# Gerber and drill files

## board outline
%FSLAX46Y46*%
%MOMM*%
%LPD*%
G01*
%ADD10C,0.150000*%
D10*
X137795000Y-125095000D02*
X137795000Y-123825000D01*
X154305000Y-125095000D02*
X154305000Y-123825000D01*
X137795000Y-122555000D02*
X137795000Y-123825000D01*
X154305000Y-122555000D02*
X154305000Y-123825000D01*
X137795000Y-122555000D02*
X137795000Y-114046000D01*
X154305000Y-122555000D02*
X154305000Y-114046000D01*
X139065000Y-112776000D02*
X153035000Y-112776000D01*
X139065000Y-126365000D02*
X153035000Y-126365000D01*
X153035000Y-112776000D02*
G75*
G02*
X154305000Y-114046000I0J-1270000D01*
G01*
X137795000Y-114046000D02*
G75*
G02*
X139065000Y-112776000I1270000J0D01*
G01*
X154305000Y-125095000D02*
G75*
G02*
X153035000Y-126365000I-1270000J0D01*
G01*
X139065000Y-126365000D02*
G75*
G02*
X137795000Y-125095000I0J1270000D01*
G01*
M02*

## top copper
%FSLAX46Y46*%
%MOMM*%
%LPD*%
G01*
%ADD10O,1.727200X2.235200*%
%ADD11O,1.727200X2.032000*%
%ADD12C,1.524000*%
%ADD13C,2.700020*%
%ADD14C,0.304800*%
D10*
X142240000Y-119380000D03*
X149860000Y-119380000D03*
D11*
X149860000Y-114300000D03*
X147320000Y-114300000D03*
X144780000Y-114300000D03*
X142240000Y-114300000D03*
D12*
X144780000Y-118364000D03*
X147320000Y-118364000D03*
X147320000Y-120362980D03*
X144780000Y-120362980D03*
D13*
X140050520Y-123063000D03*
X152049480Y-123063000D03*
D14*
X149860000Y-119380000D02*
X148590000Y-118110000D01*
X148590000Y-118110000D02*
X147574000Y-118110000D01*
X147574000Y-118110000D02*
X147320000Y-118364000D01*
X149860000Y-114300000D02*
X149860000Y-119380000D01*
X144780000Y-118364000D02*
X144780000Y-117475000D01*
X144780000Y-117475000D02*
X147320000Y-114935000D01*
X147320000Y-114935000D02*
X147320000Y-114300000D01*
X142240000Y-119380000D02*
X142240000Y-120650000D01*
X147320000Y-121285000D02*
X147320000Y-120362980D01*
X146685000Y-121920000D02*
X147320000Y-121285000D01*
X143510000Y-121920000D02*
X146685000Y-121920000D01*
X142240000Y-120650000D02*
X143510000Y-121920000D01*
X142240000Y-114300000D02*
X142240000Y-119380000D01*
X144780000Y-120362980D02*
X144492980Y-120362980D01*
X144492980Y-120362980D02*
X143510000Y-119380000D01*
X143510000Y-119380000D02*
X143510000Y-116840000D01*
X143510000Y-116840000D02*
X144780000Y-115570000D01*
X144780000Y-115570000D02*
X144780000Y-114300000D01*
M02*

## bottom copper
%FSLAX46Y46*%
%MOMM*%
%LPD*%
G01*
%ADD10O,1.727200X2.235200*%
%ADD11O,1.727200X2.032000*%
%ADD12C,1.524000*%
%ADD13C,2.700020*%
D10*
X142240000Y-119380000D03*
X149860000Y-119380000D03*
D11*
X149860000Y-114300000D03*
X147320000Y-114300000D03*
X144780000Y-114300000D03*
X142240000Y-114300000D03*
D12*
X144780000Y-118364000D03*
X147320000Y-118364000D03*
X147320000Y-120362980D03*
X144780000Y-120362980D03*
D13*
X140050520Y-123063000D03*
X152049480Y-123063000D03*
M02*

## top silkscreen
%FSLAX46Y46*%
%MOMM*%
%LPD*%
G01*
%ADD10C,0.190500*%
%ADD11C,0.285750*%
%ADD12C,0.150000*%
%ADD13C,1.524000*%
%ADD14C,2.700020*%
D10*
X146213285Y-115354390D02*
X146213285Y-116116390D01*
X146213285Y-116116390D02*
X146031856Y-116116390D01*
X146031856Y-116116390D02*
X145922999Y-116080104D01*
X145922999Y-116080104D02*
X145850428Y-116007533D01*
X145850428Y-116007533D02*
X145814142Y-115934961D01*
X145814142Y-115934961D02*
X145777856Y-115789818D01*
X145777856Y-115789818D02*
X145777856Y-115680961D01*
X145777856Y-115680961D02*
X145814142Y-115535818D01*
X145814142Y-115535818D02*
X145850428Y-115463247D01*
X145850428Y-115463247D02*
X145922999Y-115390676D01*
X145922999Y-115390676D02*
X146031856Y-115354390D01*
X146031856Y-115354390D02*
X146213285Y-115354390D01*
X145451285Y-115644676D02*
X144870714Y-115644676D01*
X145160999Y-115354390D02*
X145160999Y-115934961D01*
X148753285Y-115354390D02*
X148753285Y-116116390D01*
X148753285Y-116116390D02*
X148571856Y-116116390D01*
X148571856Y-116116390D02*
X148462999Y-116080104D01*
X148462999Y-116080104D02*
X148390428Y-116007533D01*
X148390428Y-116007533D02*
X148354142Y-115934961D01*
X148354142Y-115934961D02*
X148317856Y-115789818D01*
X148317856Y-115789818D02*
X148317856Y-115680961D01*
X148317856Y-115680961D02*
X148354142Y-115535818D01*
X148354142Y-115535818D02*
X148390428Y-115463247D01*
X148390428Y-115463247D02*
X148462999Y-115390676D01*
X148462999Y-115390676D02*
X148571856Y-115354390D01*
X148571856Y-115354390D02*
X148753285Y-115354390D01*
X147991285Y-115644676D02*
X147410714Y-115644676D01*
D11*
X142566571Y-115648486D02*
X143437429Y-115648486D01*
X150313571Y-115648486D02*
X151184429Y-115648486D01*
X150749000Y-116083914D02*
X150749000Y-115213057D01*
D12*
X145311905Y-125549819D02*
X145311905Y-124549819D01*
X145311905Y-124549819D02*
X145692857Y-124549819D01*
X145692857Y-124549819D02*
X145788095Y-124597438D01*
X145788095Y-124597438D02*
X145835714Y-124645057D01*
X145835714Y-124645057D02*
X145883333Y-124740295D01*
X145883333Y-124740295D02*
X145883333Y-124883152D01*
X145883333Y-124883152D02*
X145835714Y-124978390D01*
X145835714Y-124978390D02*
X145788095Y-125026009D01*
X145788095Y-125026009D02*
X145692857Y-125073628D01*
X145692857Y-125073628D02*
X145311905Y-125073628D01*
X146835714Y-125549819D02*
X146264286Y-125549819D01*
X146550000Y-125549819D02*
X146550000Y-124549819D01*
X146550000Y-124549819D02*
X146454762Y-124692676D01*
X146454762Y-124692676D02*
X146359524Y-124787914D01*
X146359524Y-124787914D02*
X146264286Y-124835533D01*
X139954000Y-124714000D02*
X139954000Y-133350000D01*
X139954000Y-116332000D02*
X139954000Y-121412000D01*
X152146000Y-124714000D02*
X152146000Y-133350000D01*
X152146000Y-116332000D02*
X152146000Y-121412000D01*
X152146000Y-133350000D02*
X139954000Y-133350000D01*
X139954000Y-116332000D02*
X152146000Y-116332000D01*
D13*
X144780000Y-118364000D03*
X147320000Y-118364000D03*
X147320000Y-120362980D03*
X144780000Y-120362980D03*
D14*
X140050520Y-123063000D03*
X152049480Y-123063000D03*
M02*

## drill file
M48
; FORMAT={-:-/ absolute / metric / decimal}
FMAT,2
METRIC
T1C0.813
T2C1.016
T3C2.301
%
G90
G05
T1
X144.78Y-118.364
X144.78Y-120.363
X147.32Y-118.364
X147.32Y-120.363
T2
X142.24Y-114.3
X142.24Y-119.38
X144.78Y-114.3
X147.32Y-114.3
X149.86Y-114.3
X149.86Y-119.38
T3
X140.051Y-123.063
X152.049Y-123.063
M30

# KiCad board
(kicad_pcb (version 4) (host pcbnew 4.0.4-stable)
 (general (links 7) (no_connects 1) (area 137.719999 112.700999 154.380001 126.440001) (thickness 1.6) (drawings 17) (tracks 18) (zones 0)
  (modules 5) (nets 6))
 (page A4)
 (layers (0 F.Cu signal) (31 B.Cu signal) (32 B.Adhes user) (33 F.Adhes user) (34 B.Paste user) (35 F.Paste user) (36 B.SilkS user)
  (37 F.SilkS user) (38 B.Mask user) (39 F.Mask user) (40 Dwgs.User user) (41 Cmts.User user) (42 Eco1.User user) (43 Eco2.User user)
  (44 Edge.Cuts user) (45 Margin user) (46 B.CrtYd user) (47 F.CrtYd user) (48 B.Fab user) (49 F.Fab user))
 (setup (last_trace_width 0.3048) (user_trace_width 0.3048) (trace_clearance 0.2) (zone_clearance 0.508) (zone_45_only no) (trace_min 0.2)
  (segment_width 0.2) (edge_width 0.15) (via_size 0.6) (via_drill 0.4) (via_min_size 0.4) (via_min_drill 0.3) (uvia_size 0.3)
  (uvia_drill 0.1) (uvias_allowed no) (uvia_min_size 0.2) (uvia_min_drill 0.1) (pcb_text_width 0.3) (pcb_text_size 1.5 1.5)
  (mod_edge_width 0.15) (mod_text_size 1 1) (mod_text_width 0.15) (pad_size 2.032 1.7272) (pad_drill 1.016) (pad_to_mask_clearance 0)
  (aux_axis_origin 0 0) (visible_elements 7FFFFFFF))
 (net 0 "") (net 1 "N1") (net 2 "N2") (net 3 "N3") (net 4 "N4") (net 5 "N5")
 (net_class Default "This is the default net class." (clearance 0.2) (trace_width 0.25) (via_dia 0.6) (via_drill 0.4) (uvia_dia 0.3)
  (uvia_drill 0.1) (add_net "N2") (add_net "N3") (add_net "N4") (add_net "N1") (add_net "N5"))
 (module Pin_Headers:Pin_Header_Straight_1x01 (layer B.Cu) (at 142.24 119.38)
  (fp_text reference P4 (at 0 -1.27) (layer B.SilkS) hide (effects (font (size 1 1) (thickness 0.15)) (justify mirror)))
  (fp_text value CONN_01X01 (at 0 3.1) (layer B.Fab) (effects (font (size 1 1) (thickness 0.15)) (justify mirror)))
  (pad 1 thru_hole oval (at 0 0) (size 1.7272 2.2352) (drill 1.016) (layers *.Cu *.Mask B.SilkS) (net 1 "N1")))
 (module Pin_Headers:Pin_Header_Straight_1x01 (layer B.Cu) (at 149.86 119.38)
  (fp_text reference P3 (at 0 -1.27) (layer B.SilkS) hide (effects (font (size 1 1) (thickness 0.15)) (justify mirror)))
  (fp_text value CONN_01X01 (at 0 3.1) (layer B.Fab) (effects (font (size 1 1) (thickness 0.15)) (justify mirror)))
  (pad 1 thru_hole oval (at 0 0) (size 1.7272 2.2352) (drill 1.016) (layers *.Cu *.Mask B.SilkS) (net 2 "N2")))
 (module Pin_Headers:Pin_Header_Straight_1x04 (layer B.Cu) (at 149.86 114.3 90)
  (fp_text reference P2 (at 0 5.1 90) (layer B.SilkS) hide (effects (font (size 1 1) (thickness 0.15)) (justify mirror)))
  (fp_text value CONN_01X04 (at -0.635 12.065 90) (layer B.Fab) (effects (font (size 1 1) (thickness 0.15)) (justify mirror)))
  (pad 1 thru_hole oval (at 0 0 90) (size 2.032 1.7272) (drill 1.016) (layers *.Cu *.Mask B.SilkS) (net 2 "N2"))
  (pad 2 thru_hole oval (at 0 -2.54 90) (size 2.032 1.7272) (drill 1.016) (layers *.Cu *.Mask B.SilkS) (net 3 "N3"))
  (pad 3 thru_hole oval (at 0 -5.08 90) (size 2.032 1.7272) (drill 1.016) (layers *.Cu *.Mask B.SilkS) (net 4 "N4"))
  (pad 4 thru_hole oval (at 0 -7.62 90) (size 2.032 1.7272) (drill 1.016) (layers *.Cu *.Mask B.SilkS) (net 1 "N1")))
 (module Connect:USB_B (layer F.Cu) (at 147.32 118.364 270)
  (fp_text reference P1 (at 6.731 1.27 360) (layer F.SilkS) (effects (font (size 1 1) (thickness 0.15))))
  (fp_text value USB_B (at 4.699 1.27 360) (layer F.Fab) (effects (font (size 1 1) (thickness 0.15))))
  (fp_line (start 6.35 7.366) (end 14.986 7.366) (layer F.SilkS) (width 0.15))
  (fp_line (start -2.032 7.366) (end 3.048 7.366) (layer F.SilkS) (width 0.15))
  (fp_line (start 6.35 -4.826) (end 14.986 -4.826) (layer F.SilkS) (width 0.15))
  (fp_line (start -2.032 -4.826) (end 3.048 -4.826) (layer F.SilkS) (width 0.15))
  (fp_line (start 14.986 -4.826) (end 14.986 7.366) (layer F.SilkS) (width 0.15))
  (fp_line (start -2.032 7.366) (end -2.032 -4.826) (layer F.SilkS) (width 0.15))
  (pad 2 thru_hole circle (at 0 2.54 180) (size 1.524 1.524) (drill 0.8128) (layers *.Cu *.Mask F.SilkS) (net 3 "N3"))
  (pad 1 thru_hole circle (at 0 0 180) (size 1.524 1.524) (drill 0.8128) (layers *.Cu *.Mask F.SilkS) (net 2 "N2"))
  (pad 4 thru_hole circle (at 1.99898 0 180) (size 1.524 1.524) (drill 0.8128) (layers *.Cu *.Mask F.SilkS) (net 1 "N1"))
  (pad 3 thru_hole circle (at 1.99898 2.54 180) (size 1.524 1.524) (drill 0.8128) (layers *.Cu *.Mask F.SilkS) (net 4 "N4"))
  (pad 5 thru_hole circle (at 4.699 7.26948 180) (size 2.70002 2.70002) (drill 2.30124) (layers *.Cu *.Mask F.SilkS) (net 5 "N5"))
  (pad 5 thru_hole circle (at 4.699 -4.72948 180) (size 2.70002 2.70002) (drill 2.30124) (layers *.Cu *.Mask F.SilkS) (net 5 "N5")))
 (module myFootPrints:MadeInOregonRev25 (layer F.Cu) (at 146.05 123.825)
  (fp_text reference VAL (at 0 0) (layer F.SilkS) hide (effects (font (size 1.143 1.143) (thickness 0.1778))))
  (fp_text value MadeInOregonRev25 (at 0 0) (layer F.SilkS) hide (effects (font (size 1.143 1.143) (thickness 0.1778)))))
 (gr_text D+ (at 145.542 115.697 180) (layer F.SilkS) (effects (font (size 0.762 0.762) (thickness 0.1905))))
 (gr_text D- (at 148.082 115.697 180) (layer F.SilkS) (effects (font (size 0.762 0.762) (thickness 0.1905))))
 (gr_line (start 137.795 125.095) (end 137.795 123.825) (angle 90) (layer Edge.Cuts) (width 0.15))
 (gr_line (start 154.305 125.095) (end 154.305 123.825) (angle 90) (layer Edge.Cuts) (width 0.15))
 (gr_line (start 137.795 122.555) (end 137.795 123.825) (angle 90) (layer Edge.Cuts) (width 0.15))
 (gr_line (start 154.305 122.555) (end 154.305 123.825) (angle 90) (layer Edge.Cuts) (width 0.15))
 (gr_line (start 137.795 122.555) (end 137.795 114.046) (angle 90) (layer Edge.Cuts) (width 0.15))
 (gr_line (start 154.305 122.555) (end 154.305 114.046) (angle 90) (layer Edge.Cuts) (width 0.15))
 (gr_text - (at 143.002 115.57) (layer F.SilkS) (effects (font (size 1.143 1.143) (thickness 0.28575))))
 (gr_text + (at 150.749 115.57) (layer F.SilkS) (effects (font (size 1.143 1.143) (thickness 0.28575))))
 (gr_line (start 139.065 112.776) (end 153.035 112.776) (angle 90) (layer Edge.Cuts) (width 0.15))
 (gr_line (start 139.065 126.365) (end 153.035 126.365) (angle 90) (layer Edge.Cuts) (width 0.15))
 (gr_arc (start 153.035 114.046) (end 153.035 112.776) (angle 90) (layer Edge.Cuts) (width 0.15))
 (gr_arc (start 139.065 114.046) (end 137.795 114.046) (angle 90) (layer Edge.Cuts) (width 0.15))
 (gr_arc (start 153.035 125.095) (end 154.305 125.095) (angle 90) (layer Edge.Cuts) (width 0.15))
 (gr_arc (start 139.065 125.095) (end 139.065 126.365) (angle 90) (layer Edge.Cuts) (width 0.15))
 (segment (start 149.86 119.38) (end 148.59 118.11) (width 0.3048) (layer F.Cu) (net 2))
 (segment (start 148.59 118.11) (end 147.574 118.11) (width 0.3048) (layer F.Cu) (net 2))
 (segment (start 147.574 118.11) (end 147.32 118.364) (width 0.3048) (layer F.Cu) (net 2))
 (segment (start 149.86 114.3) (end 149.86 119.38) (width 0.3048) (layer F.Cu) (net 2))
 (segment (start 144.78 118.364) (end 144.78 117.475) (width 0.3048) (layer F.Cu) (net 3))
 (segment (start 144.78 117.475) (end 147.32 114.935) (width 0.3048) (layer F.Cu) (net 3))
 (segment (start 147.32 114.935) (end 147.32 114.3) (width 0.3048) (layer F.Cu) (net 3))
 (segment (start 142.24 119.38) (end 142.24 120.65) (width 0.3048) (layer F.Cu) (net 1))
 (segment (start 147.32 121.285) (end 147.32 120.36298) (width 0.3048) (layer F.Cu) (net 1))
 (segment (start 146.685 121.92) (end 147.32 121.285) (width 0.3048) (layer F.Cu) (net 1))
 (segment (start 143.51 121.92) (end 146.685 121.92) (width 0.3048) (layer F.Cu) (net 1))
 (segment (start 142.24 120.65) (end 143.51 121.92) (width 0.3048) (layer F.Cu) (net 1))
 (segment (start 142.24 114.3) (end 142.24 119.38) (width 0.3048) (layer F.Cu) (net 1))
 (segment (start 144.78 120.36298) (end 144.49298 120.36298) (width 0.3048) (layer F.Cu) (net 4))
 (segment (start 144.49298 120.36298) (end 143.51 119.38) (width 0.3048) (layer F.Cu) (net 4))
 (segment (start 143.51 119.38) (end 143.51 116.84) (width 0.3048) (layer F.Cu) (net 4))
 (segment (start 143.51 116.84) (end 144.78 115.57) (width 0.3048) (layer F.Cu) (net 4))
 (segment (start 144.78 115.57) (end 144.78 114.3) (width 0.3048) (layer F.Cu) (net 4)))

